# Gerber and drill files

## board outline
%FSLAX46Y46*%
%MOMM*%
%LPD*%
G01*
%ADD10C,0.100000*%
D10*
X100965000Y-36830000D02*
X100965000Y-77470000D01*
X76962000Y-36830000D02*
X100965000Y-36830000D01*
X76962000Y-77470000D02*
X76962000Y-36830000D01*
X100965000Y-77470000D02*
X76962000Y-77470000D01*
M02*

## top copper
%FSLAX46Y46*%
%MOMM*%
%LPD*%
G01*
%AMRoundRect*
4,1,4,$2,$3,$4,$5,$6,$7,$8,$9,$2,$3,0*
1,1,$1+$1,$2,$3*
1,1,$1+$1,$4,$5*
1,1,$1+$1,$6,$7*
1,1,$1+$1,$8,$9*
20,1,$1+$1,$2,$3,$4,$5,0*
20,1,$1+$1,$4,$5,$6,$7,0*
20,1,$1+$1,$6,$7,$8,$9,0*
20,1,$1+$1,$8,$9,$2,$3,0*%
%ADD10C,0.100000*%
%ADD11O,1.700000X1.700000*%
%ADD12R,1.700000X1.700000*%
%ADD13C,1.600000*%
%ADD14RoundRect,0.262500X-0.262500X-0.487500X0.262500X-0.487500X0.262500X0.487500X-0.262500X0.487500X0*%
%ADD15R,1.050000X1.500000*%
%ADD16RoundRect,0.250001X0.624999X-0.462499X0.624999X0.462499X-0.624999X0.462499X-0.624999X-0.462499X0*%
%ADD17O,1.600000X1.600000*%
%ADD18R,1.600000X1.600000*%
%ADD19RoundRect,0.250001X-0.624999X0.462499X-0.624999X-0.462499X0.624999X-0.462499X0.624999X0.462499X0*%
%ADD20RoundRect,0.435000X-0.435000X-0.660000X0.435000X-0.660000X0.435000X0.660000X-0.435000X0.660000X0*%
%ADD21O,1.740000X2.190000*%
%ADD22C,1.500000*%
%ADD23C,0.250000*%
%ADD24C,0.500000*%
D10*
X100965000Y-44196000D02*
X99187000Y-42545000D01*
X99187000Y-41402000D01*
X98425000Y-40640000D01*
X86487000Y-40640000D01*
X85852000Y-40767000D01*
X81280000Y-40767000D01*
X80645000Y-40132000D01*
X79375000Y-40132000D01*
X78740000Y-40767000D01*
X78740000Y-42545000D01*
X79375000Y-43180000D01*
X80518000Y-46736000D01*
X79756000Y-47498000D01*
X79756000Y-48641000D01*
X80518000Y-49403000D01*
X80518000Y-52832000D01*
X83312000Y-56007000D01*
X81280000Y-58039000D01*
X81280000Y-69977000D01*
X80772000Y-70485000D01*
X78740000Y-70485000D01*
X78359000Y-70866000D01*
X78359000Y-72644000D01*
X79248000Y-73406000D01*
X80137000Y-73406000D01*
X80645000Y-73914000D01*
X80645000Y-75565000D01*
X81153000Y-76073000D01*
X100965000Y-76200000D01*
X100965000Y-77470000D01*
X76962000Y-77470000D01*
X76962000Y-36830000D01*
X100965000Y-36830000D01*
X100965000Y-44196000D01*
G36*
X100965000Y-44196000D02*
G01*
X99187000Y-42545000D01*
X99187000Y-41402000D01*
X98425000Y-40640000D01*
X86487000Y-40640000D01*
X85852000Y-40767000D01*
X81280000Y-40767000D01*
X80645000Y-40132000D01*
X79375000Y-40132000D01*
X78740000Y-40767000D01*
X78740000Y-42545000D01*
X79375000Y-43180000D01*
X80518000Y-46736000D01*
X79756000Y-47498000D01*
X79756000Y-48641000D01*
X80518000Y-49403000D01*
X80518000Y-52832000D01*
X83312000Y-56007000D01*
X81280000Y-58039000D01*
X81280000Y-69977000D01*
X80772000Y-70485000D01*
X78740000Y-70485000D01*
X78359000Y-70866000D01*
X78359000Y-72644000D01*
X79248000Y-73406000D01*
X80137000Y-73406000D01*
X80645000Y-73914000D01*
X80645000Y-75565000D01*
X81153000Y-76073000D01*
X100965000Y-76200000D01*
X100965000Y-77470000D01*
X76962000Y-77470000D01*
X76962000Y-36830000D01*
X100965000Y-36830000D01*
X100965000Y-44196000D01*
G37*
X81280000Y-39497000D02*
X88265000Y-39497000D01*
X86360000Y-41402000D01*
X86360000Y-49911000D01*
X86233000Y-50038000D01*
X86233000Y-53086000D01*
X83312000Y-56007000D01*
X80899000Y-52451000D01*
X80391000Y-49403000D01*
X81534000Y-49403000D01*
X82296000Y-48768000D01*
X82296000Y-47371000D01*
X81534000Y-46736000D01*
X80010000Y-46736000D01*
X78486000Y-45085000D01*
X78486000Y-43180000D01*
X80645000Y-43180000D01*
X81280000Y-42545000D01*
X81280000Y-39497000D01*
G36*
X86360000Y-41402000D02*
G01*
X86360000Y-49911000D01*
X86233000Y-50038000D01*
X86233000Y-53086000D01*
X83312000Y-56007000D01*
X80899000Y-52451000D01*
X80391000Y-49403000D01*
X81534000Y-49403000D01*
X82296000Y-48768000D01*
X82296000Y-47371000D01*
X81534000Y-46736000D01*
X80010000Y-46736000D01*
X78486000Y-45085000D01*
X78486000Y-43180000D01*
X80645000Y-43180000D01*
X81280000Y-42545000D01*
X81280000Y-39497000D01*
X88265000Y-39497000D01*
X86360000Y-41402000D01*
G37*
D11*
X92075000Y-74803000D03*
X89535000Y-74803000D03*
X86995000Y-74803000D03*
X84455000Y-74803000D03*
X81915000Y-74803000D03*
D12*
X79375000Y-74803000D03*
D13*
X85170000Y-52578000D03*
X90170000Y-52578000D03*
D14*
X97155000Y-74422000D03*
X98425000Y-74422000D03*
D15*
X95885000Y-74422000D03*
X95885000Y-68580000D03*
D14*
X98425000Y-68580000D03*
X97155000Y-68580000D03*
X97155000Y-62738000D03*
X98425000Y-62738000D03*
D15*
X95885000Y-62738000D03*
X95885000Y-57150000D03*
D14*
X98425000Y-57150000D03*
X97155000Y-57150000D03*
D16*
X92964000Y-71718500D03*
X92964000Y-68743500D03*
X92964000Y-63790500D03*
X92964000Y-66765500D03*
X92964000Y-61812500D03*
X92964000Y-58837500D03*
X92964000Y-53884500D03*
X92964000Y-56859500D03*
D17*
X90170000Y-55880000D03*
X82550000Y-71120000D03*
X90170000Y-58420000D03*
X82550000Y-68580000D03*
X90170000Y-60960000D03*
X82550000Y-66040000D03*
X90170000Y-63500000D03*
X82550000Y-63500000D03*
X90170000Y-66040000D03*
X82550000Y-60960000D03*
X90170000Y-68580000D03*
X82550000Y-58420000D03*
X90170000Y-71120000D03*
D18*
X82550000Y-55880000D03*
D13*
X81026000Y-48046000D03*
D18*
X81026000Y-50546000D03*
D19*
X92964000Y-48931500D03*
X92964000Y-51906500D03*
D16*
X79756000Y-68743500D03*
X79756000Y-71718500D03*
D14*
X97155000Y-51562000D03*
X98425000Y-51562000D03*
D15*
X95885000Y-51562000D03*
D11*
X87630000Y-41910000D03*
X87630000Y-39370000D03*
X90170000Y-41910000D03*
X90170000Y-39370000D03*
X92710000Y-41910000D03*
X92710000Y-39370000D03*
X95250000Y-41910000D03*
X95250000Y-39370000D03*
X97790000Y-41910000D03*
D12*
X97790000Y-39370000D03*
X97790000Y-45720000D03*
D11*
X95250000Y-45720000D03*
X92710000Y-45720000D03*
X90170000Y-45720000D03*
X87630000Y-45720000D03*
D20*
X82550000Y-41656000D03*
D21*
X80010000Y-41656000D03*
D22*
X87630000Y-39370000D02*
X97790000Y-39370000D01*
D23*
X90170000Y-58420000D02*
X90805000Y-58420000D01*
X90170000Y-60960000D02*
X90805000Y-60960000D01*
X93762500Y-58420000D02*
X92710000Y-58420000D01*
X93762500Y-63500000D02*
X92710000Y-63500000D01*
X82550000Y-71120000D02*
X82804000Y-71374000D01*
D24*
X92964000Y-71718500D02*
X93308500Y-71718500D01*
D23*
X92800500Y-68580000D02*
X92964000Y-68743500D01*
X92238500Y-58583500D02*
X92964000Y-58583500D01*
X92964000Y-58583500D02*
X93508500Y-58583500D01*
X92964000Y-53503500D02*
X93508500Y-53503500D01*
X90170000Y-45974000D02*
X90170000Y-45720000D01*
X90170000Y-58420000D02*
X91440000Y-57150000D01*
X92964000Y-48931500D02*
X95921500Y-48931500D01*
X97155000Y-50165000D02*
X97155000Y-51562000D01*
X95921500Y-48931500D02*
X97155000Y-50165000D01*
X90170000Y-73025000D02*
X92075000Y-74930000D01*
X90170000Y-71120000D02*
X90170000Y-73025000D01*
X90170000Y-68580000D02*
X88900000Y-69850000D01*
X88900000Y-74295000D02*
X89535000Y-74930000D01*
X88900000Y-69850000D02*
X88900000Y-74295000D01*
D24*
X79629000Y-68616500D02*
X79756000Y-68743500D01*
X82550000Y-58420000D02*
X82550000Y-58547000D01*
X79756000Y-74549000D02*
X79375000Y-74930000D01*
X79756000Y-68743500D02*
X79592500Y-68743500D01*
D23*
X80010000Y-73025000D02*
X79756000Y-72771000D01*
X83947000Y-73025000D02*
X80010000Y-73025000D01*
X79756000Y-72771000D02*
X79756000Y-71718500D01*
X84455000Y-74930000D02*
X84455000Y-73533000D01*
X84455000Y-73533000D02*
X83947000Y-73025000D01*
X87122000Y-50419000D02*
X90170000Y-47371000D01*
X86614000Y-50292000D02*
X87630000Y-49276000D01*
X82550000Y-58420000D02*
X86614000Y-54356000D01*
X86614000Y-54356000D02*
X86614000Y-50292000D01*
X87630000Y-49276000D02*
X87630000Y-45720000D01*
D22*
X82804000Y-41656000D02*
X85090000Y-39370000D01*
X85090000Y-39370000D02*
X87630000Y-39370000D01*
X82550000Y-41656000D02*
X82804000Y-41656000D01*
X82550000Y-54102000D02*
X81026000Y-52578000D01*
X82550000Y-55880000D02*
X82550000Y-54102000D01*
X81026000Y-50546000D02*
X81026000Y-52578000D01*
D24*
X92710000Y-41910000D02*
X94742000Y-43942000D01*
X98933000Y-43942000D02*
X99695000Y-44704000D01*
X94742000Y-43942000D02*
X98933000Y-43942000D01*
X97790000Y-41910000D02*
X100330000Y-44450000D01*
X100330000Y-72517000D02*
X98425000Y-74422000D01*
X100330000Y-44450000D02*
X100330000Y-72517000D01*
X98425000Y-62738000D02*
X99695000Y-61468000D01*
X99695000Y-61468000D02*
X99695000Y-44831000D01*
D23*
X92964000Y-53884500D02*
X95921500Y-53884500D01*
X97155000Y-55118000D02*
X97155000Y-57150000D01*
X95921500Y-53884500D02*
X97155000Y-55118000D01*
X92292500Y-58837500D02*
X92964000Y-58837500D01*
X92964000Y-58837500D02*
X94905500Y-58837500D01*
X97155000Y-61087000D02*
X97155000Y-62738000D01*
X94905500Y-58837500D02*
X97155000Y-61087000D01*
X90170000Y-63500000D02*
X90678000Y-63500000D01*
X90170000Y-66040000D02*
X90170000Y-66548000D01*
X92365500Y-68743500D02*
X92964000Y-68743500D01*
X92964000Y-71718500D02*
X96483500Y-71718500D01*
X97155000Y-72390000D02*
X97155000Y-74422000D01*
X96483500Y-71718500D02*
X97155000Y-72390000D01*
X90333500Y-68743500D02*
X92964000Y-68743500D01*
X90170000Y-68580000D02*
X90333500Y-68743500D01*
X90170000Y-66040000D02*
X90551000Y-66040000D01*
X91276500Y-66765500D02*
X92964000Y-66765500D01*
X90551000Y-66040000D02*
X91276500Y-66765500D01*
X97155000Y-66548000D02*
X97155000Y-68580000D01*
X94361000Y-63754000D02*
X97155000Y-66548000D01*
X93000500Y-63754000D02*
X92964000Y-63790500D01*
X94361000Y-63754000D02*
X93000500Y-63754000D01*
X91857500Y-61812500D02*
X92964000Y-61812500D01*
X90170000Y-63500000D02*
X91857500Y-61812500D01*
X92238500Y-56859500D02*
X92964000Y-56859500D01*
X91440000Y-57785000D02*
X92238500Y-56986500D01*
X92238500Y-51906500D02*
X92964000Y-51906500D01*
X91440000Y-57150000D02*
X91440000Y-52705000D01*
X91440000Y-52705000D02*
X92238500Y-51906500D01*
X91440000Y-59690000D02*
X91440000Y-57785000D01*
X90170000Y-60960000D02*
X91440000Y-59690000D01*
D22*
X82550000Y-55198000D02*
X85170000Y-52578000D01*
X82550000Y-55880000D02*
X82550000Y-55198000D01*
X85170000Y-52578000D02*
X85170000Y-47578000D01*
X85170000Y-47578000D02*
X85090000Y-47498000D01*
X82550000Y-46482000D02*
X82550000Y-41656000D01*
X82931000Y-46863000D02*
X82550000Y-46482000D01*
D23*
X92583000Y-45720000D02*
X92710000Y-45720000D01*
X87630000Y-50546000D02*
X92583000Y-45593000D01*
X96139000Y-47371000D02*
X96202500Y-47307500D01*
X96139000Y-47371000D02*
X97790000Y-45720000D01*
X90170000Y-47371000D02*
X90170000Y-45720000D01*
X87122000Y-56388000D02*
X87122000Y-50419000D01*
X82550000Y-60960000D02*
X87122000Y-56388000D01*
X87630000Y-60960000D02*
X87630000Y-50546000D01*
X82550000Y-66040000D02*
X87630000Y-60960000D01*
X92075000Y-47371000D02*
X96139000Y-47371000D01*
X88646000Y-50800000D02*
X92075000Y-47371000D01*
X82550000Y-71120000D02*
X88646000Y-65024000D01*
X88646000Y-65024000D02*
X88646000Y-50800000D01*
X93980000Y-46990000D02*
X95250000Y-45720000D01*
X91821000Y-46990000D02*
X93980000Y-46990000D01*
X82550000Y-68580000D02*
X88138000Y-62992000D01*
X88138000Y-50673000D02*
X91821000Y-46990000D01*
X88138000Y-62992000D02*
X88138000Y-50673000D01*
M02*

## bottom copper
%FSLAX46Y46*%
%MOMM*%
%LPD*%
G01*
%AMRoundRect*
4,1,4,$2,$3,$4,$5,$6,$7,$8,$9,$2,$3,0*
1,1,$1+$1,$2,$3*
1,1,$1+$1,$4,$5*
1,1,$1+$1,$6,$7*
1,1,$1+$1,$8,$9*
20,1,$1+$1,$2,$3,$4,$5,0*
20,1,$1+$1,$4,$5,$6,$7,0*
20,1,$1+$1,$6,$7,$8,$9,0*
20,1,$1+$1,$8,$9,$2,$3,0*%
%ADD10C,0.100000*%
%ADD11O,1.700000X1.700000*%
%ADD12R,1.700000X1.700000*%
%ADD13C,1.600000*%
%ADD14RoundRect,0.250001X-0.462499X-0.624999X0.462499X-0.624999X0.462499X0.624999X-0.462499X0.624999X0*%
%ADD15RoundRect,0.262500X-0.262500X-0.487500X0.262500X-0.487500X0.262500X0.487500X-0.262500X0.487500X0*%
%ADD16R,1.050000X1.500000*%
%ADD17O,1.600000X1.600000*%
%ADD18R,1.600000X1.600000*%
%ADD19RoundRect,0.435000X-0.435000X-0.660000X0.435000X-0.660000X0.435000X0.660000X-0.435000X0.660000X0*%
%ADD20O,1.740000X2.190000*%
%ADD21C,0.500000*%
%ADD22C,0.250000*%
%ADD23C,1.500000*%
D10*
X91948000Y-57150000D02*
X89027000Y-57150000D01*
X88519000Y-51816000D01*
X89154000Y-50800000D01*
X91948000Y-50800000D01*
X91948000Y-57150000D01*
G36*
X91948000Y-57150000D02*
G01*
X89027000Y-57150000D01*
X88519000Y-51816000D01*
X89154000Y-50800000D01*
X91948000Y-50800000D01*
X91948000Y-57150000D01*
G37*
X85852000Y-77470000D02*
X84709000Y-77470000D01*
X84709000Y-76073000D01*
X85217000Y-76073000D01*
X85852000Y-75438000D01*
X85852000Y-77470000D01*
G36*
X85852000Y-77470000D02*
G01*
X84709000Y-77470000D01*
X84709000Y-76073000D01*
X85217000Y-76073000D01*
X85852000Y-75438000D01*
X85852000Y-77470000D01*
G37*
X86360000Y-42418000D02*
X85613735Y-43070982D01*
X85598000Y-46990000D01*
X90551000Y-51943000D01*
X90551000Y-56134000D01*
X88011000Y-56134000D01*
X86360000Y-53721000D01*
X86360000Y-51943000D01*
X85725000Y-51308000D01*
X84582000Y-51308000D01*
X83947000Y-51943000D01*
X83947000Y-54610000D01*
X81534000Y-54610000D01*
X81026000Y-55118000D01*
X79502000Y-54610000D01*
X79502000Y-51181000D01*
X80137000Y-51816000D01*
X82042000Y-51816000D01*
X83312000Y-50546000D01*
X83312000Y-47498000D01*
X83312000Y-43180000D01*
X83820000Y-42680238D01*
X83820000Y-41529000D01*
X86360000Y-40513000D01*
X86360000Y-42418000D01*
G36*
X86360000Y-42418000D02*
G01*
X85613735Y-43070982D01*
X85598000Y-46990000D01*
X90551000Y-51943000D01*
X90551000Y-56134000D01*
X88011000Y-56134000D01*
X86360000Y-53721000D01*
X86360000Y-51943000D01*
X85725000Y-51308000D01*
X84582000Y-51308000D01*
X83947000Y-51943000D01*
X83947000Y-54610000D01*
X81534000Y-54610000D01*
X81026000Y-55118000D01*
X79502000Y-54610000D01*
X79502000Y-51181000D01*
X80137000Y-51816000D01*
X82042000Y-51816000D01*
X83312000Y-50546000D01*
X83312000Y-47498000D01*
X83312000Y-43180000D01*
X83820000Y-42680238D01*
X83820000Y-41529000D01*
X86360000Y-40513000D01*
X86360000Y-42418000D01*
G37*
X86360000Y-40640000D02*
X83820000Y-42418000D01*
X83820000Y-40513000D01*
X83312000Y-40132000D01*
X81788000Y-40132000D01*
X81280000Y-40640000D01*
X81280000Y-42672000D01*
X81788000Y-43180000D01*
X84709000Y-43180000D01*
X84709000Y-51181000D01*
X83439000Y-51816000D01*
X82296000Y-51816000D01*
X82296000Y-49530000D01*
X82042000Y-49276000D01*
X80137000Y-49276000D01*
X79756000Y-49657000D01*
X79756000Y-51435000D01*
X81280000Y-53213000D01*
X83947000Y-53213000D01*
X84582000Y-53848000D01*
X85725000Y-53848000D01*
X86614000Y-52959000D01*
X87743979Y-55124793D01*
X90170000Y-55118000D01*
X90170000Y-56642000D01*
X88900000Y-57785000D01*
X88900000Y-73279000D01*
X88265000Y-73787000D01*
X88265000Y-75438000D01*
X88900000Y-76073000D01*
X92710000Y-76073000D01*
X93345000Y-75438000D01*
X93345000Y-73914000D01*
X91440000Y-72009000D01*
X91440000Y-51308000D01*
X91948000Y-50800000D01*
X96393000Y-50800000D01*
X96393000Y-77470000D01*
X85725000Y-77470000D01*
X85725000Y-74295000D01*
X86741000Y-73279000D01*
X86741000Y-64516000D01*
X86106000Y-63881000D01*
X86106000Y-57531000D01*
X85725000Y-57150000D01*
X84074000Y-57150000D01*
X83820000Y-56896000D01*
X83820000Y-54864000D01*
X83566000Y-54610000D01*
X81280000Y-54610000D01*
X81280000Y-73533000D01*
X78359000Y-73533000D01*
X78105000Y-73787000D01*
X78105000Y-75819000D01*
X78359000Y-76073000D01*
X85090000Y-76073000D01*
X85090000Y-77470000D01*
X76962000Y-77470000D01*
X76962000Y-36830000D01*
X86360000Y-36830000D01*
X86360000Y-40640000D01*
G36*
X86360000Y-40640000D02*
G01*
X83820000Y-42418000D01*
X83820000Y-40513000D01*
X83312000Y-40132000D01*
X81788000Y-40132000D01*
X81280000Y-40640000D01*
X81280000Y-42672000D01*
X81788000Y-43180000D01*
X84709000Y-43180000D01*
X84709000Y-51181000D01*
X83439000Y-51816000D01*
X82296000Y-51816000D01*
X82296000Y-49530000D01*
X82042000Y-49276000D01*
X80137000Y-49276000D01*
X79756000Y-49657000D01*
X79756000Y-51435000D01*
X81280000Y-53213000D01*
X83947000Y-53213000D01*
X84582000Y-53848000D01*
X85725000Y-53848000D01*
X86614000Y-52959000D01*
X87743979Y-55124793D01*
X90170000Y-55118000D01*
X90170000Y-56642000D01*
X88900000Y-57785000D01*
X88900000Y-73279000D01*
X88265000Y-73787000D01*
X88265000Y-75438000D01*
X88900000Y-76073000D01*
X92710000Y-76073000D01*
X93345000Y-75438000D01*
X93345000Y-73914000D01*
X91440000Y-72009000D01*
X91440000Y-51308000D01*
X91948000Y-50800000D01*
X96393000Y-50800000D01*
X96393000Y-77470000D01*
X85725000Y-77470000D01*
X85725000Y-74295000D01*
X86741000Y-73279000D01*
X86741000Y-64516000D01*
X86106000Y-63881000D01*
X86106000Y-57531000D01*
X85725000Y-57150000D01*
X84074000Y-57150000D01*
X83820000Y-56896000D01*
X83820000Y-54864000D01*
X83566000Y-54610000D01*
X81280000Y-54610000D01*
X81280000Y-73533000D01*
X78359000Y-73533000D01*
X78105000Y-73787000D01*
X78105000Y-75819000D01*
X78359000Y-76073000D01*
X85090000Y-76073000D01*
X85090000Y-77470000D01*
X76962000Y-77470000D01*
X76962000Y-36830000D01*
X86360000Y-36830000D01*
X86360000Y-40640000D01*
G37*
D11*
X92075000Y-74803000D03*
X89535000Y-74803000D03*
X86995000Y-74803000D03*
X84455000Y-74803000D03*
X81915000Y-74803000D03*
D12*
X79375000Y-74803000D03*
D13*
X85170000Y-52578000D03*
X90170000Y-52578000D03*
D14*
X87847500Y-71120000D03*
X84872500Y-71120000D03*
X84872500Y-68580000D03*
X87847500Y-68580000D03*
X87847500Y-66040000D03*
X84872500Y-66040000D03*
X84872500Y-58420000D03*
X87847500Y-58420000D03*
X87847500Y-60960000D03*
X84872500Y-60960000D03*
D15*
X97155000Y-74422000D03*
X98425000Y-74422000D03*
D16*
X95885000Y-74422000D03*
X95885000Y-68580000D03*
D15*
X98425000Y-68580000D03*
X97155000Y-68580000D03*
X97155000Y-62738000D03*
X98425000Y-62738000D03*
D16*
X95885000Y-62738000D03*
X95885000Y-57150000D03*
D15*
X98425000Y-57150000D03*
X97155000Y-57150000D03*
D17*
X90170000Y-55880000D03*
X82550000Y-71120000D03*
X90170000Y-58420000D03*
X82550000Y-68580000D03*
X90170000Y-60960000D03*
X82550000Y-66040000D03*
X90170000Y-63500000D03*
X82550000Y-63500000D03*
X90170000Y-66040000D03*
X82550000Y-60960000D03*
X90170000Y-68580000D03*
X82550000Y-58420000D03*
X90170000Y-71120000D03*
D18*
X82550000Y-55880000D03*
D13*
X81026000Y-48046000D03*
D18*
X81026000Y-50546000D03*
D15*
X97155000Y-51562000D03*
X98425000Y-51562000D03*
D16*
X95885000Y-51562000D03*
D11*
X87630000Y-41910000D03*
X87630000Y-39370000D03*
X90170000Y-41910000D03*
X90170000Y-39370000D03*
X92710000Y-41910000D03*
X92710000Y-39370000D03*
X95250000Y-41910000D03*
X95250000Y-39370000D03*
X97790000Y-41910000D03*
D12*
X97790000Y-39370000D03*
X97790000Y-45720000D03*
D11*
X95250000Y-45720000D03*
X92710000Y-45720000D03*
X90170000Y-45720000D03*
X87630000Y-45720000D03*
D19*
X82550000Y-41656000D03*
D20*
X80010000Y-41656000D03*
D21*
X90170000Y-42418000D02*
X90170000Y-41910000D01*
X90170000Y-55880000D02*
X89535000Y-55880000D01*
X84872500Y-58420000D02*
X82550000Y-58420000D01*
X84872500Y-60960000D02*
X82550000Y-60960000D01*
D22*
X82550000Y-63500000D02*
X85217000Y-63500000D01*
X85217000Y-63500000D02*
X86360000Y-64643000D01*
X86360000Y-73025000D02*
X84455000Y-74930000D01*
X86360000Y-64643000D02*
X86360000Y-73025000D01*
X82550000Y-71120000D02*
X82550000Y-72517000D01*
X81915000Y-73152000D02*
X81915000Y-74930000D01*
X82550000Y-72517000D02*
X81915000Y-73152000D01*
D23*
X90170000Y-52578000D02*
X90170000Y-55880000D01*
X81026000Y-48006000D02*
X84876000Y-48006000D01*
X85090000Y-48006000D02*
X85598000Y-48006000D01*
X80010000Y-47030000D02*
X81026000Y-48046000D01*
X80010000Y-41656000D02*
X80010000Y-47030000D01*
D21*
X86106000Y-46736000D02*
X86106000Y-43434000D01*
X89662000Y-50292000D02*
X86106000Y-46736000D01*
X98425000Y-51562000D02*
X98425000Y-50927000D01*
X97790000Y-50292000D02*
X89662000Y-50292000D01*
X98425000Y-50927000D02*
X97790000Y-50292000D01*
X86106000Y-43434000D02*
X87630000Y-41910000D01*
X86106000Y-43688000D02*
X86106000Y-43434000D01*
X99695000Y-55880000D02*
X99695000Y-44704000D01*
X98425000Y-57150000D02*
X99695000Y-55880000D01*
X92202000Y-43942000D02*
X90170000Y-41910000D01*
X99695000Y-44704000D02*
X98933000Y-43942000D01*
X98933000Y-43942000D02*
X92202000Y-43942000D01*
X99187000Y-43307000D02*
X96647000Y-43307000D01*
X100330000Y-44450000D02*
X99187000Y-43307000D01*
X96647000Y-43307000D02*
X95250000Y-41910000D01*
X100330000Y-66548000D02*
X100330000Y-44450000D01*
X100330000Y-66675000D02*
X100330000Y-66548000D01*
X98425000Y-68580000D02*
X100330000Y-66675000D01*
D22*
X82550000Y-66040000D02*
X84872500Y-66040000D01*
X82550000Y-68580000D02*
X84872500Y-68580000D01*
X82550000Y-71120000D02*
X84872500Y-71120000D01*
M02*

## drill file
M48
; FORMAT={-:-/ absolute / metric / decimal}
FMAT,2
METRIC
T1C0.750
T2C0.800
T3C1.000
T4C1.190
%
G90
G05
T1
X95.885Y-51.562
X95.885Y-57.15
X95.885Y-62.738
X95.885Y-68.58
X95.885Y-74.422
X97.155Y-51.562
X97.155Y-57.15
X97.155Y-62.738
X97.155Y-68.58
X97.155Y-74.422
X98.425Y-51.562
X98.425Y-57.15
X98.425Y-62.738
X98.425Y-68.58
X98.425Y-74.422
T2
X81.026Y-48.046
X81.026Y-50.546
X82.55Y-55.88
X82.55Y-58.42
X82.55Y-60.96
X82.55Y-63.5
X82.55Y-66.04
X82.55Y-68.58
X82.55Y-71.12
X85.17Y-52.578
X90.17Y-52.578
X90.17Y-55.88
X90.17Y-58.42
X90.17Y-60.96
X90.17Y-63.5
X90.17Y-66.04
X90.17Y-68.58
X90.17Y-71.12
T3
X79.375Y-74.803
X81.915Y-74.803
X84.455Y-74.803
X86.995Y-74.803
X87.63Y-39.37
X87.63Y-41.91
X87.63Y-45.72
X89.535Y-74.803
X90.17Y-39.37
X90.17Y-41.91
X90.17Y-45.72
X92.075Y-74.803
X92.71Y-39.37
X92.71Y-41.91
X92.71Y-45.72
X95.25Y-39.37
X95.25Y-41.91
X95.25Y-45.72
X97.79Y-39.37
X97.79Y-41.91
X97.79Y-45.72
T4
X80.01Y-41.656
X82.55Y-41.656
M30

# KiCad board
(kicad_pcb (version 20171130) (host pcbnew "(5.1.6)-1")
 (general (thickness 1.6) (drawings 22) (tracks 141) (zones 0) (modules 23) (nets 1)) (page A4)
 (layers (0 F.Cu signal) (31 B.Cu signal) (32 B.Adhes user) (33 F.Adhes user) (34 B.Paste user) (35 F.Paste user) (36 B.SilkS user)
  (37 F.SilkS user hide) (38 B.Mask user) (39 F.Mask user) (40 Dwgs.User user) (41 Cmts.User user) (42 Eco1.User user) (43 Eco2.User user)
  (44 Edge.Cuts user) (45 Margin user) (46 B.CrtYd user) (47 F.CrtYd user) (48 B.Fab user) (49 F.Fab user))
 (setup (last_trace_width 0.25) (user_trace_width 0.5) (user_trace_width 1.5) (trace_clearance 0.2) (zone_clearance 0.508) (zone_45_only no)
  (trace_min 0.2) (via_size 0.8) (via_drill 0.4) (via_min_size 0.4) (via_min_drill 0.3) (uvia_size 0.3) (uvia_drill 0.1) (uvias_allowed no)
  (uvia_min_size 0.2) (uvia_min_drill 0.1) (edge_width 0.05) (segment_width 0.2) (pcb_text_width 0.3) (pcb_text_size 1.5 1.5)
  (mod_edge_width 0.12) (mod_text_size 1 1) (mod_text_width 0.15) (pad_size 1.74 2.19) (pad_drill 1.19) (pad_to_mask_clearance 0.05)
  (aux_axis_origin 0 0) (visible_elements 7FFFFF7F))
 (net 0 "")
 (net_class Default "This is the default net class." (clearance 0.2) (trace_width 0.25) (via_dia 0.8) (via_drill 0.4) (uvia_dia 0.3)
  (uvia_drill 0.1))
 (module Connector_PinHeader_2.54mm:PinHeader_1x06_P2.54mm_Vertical (layer F.Cu) (at 79.375 74.803 90)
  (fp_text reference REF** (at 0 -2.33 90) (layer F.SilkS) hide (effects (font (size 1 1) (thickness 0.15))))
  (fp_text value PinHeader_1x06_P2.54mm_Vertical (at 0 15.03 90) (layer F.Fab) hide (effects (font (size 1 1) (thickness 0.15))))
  (pad 6 thru_hole oval (at 0 12.7 90) (size 1.7 1.7) (drill 1) (layers *.Cu *.Mask))
  (pad 5 thru_hole oval (at 0 10.16 90) (size 1.7 1.7) (drill 1) (layers *.Cu *.Mask))
  (pad 4 thru_hole oval (at 0 7.62 90) (size 1.7 1.7) (drill 1) (layers *.Cu *.Mask))
  (pad 3 thru_hole oval (at 0 5.08 90) (size 1.7 1.7) (drill 1) (layers *.Cu *.Mask))
  (pad 2 thru_hole oval (at 0 2.54 90) (size 1.7 1.7) (drill 1) (layers *.Cu *.Mask))
  (pad 1 thru_hole rect (at 0 0 90) (size 1.7 1.7) (drill 1) (layers *.Cu *.Mask)))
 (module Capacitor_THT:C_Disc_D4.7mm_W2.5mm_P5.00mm (layer F.Cu) (at 90.17 52.578 180)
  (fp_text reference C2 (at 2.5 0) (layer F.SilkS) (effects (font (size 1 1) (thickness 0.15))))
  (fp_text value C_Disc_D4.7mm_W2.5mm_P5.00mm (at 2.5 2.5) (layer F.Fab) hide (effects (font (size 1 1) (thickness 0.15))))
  (pad 2 thru_hole circle (at 5 0 180) (size 1.6 1.6) (drill 0.8) (layers *.Cu *.Mask))
  (pad 1 thru_hole circle (at 0 0 180) (size 1.6 1.6) (drill 0.8) (layers *.Cu *.Mask)))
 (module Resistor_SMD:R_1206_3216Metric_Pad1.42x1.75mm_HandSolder (layer B.Cu) (at 86.36 71.12)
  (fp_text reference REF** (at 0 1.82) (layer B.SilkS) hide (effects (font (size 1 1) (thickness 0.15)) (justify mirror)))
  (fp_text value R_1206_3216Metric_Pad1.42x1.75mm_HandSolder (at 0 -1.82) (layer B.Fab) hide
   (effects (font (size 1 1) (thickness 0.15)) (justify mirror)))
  (pad 2 smd roundrect (at 1.4875 0) (size 1.425 1.75) (layers B.Cu B.Paste B.Mask) (roundrect_rratio 0.175439))
  (pad 1 smd roundrect (at -1.4875 0) (size 1.425 1.75) (layers B.Cu B.Paste B.Mask) (roundrect_rratio 0.175439)))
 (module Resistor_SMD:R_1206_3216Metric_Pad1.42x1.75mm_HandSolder (layer B.Cu) (at 86.36 68.58)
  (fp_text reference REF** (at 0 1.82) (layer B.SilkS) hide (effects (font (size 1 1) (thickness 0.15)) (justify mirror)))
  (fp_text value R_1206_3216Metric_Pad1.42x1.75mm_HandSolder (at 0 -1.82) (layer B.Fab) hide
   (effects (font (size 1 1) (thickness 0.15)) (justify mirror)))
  (pad 1 smd roundrect (at -1.4875 0) (size 1.425 1.75) (layers B.Cu B.Paste B.Mask) (roundrect_rratio 0.175439))
  (pad 2 smd roundrect (at 1.4875 0) (size 1.425 1.75) (layers B.Cu B.Paste B.Mask) (roundrect_rratio 0.175439)))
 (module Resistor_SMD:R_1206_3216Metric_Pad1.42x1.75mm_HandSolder (layer B.Cu) (at 86.36 66.04)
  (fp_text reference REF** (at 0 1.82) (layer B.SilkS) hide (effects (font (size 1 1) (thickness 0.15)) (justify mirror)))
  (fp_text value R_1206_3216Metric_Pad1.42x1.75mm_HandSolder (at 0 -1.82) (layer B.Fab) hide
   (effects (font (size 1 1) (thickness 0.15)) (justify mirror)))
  (pad 2 smd roundrect (at 1.4875 0) (size 1.425 1.75) (layers B.Cu B.Paste B.Mask) (roundrect_rratio 0.175439))
  (pad 1 smd roundrect (at -1.4875 0) (size 1.425 1.75) (layers B.Cu B.Paste B.Mask) (roundrect_rratio 0.175439)))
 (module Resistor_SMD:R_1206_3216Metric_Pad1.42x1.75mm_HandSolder (layer B.Cu) (at 86.36 58.42)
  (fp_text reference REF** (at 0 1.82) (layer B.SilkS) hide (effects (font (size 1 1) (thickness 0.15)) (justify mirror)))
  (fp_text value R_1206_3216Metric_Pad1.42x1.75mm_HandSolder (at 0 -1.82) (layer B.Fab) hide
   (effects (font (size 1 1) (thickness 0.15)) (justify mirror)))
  (pad 1 smd roundrect (at -1.4875 0) (size 1.425 1.75) (layers B.Cu B.Paste B.Mask) (roundrect_rratio 0.175439))
  (pad 2 smd roundrect (at 1.4875 0) (size 1.425 1.75) (layers B.Cu B.Paste B.Mask) (roundrect_rratio 0.175439)))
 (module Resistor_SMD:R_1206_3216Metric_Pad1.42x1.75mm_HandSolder (layer B.Cu) (at 86.36 60.96)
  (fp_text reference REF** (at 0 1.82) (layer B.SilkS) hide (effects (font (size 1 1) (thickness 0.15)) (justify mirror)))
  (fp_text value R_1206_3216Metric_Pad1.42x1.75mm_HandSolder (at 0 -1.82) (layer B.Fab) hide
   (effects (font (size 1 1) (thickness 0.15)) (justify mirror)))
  (pad 2 smd roundrect (at 1.4875 0) (size 1.425 1.75) (layers B.Cu B.Paste B.Mask) (roundrect_rratio 0.175439))
  (pad 1 smd roundrect (at -1.4875 0) (size 1.425 1.75) (layers B.Cu B.Paste B.Mask) (roundrect_rratio 0.175439)))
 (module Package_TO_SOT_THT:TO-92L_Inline (layer F.Cu) (at 95.885 74.422)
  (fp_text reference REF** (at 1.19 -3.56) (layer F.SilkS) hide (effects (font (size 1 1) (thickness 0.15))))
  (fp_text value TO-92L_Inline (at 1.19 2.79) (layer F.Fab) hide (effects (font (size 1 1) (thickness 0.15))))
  (pad 2 thru_hole roundrect (at 1.27 0) (size 1.05 1.5) (drill 0.75) (layers *.Cu *.Mask) (roundrect_rratio 0.25))
  (pad 3 thru_hole roundrect (at 2.54 0) (size 1.05 1.5) (drill 0.75) (layers *.Cu *.Mask) (roundrect_rratio 0.25))
  (pad 1 thru_hole rect (at 0 0) (size 1.05 1.5) (drill 0.75) (layers *.Cu *.Mask)))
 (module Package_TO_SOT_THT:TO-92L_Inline (layer F.Cu) (at 95.885 68.58)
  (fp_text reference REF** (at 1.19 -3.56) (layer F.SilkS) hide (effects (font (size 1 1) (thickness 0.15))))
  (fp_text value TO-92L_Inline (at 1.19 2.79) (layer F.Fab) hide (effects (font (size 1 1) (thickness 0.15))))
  (pad 1 thru_hole rect (at 0 0) (size 1.05 1.5) (drill 0.75) (layers *.Cu *.Mask))
  (pad 3 thru_hole roundrect (at 2.54 0) (size 1.05 1.5) (drill 0.75) (layers *.Cu *.Mask) (roundrect_rratio 0.25))
  (pad 2 thru_hole roundrect (at 1.27 0) (size 1.05 1.5) (drill 0.75) (layers *.Cu *.Mask) (roundrect_rratio 0.25)))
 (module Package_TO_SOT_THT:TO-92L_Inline (layer F.Cu) (at 95.885 62.738)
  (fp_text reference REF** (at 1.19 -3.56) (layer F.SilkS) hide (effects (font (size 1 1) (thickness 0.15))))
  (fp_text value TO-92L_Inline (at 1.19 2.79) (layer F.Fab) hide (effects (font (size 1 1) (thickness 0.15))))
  (pad 2 thru_hole roundrect (at 1.27 0) (size 1.05 1.5) (drill 0.75) (layers *.Cu *.Mask) (roundrect_rratio 0.25))
  (pad 3 thru_hole roundrect (at 2.54 0) (size 1.05 1.5) (drill 0.75) (layers *.Cu *.Mask) (roundrect_rratio 0.25))
  (pad 1 thru_hole rect (at 0 0) (size 1.05 1.5) (drill 0.75) (layers *.Cu *.Mask)))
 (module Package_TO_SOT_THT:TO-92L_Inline (layer F.Cu) (at 95.885 57.15)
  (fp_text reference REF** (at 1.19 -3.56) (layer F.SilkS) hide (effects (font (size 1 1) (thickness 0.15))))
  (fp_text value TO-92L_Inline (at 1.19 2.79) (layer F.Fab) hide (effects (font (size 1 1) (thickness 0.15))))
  (pad 1 thru_hole rect (at 0 0) (size 1.05 1.5) (drill 0.75) (layers *.Cu *.Mask))
  (pad 3 thru_hole roundrect (at 2.54 0) (size 1.05 1.5) (drill 0.75) (layers *.Cu *.Mask) (roundrect_rratio 0.25))
  (pad 2 thru_hole roundrect (at 1.27 0) (size 1.05 1.5) (drill 0.75) (layers *.Cu *.Mask) (roundrect_rratio 0.25)))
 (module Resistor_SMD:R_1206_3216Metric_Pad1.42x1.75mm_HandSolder (layer F.Cu) (at 92.964 70.231 90)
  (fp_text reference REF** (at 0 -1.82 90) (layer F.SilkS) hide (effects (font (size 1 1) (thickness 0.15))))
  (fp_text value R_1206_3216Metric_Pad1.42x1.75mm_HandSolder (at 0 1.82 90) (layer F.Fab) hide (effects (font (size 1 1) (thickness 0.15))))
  (pad 1 smd roundrect (at -1.4875 0 90) (size 1.425 1.75) (layers F.Cu F.Paste F.Mask) (roundrect_rratio 0.175439))
  (pad 2 smd roundrect (at 1.4875 0 90) (size 1.425 1.75) (layers F.Cu F.Paste F.Mask) (roundrect_rratio 0.175439)))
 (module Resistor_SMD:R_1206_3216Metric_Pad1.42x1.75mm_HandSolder (layer F.Cu) (at 92.964 65.278 90)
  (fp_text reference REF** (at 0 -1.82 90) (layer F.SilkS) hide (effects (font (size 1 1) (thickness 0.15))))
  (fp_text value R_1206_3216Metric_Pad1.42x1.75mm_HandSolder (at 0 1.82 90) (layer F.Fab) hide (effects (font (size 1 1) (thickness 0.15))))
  (pad 2 smd roundrect (at 1.4875 0 90) (size 1.425 1.75) (layers F.Cu F.Paste F.Mask) (roundrect_rratio 0.175439))
  (pad 1 smd roundrect (at -1.4875 0 90) (size 1.425 1.75) (layers F.Cu F.Paste F.Mask) (roundrect_rratio 0.175439)))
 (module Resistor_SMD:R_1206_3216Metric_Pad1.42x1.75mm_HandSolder (layer F.Cu) (at 92.964 60.325 90)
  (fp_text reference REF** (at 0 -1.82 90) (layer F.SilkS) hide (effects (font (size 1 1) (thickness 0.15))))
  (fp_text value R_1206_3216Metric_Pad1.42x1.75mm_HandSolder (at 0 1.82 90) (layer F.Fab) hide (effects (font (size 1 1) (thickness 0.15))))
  (pad 1 smd roundrect (at -1.4875 0 90) (size 1.425 1.75) (layers F.Cu F.Paste F.Mask) (roundrect_rratio 0.175439))
  (pad 2 smd roundrect (at 1.4875 0 90) (size 1.425 1.75) (layers F.Cu F.Paste F.Mask) (roundrect_rratio 0.175439)))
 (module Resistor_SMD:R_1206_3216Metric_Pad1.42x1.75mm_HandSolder (layer F.Cu) (at 92.964 55.372 90)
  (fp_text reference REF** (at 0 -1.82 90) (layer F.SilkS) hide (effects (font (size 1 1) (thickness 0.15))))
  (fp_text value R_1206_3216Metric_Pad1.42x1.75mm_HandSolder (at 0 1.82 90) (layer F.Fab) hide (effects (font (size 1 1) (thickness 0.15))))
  (pad 2 smd roundrect (at 1.4875 0 90) (size 1.425 1.75) (layers F.Cu F.Paste F.Mask) (roundrect_rratio 0.175439))
  (pad 1 smd roundrect (at -1.4875 0 90) (size 1.425 1.75) (layers F.Cu F.Paste F.Mask) (roundrect_rratio 0.175439)))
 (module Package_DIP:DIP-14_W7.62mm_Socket (layer F.Cu) (at 82.55 55.88)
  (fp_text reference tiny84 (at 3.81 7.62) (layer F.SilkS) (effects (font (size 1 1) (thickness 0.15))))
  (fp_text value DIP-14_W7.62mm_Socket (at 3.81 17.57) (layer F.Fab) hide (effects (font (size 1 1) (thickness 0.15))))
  (pad 14 thru_hole oval (at 7.62 0) (size 1.6 1.6) (drill 0.8) (layers *.Cu *.Mask))
  (pad 7 thru_hole oval (at 0 15.24) (size 1.6 1.6) (drill 0.8) (layers *.Cu *.Mask))
  (pad 13 thru_hole oval (at 7.62 2.54) (size 1.6 1.6) (drill 0.8) (layers *.Cu *.Mask))
  (pad 6 thru_hole oval (at 0 12.7) (size 1.6 1.6) (drill 0.8) (layers *.Cu *.Mask))
  (pad 12 thru_hole oval (at 7.62 5.08) (size 1.6 1.6) (drill 0.8) (layers *.Cu *.Mask))
  (pad 5 thru_hole oval (at 0 10.16) (size 1.6 1.6) (drill 0.8) (layers *.Cu *.Mask))
  (pad 11 thru_hole oval (at 7.62 7.62) (size 1.6 1.6) (drill 0.8) (layers *.Cu *.Mask))
  (pad 4 thru_hole oval (at 0 7.62) (size 1.6 1.6) (drill 0.8) (layers *.Cu *.Mask))
  (pad 10 thru_hole oval (at 7.62 10.16) (size 1.6 1.6) (drill 0.8) (layers *.Cu *.Mask))
  (pad 3 thru_hole oval (at 0 5.08) (size 1.6 1.6) (drill 0.8) (layers *.Cu *.Mask))
  (pad 9 thru_hole oval (at 7.62 12.7) (size 1.6 1.6) (drill 0.8) (layers *.Cu *.Mask))
  (pad 2 thru_hole oval (at 0 2.54) (size 1.6 1.6) (drill 0.8) (layers *.Cu *.Mask))
  (pad 8 thru_hole oval (at 7.62 15.24) (size 1.6 1.6) (drill 0.8) (layers *.Cu *.Mask))
  (pad 1 thru_hole rect (at 0 0) (size 1.6 1.6) (drill 0.8) (layers *.Cu *.Mask)))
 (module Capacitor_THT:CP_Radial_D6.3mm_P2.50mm (layer F.Cu) (at 81.026 50.546 90)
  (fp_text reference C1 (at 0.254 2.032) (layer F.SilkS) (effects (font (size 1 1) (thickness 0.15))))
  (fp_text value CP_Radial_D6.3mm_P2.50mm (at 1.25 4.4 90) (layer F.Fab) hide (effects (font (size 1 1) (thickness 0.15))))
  (pad 2 thru_hole circle (at 2.5 0 90) (size 1.6 1.6) (drill 0.8) (layers *.Cu *.Mask))
  (pad 1 thru_hole rect (at 0 0 90) (size 1.6 1.6) (drill 0.8) (layers *.Cu *.Mask)))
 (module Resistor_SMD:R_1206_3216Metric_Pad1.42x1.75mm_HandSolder (layer F.Cu) (at 92.964 50.419 270)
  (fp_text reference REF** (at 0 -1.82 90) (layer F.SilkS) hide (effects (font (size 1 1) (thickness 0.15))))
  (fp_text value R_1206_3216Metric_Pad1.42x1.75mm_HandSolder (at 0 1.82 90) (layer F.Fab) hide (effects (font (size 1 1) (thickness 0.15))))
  (pad 1 smd roundrect (at -1.4875 0 270) (size 1.425 1.75) (layers F.Cu F.Paste F.Mask) (roundrect_rratio 0.175439))
  (pad 2 smd roundrect (at 1.4875 0 270) (size 1.425 1.75) (layers F.Cu F.Paste F.Mask) (roundrect_rratio 0.175439)))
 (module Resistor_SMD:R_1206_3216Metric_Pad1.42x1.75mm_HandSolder (layer F.Cu) (at 79.756 70.231 90)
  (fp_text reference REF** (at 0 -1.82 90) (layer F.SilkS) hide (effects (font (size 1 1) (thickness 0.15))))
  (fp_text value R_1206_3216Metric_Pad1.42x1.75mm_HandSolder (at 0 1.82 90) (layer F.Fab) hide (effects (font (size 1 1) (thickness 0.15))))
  (pad 2 smd roundrect (at 1.4875 0 90) (size 1.425 1.75) (layers F.Cu F.Paste F.Mask) (roundrect_rratio 0.175439))
  (pad 1 smd roundrect (at -1.4875 0 90) (size 1.425 1.75) (layers F.Cu F.Paste F.Mask) (roundrect_rratio 0.175439)))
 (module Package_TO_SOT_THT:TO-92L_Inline (layer F.Cu) (at 95.885 51.562)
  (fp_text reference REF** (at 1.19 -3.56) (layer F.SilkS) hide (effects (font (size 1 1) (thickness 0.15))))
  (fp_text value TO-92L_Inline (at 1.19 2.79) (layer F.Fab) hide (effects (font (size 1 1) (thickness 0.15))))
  (pad 2 thru_hole roundrect (at 1.27 0) (size 1.05 1.5) (drill 0.75) (layers *.Cu *.Mask) (roundrect_rratio 0.25))
  (pad 3 thru_hole roundrect (at 2.54 0) (size 1.05 1.5) (drill 0.75) (layers *.Cu *.Mask) (roundrect_rratio 0.25))
  (pad 1 thru_hole rect (at 0 0) (size 1.05 1.5) (drill 0.75) (layers *.Cu *.Mask)))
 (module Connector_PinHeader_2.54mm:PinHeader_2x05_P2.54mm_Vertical (layer F.Cu) (at 97.79 39.37 270)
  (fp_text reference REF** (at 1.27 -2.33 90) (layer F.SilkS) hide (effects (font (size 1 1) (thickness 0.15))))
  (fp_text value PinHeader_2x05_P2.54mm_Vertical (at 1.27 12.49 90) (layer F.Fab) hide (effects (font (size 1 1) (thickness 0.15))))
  (pad 10 thru_hole oval (at 2.54 10.16 270) (size 1.7 1.7) (drill 1) (layers *.Cu *.Mask))
  (pad 9 thru_hole oval (at 0 10.16 270) (size 1.7 1.7) (drill 1) (layers *.Cu *.Mask))
  (pad 8 thru_hole oval (at 2.54 7.62 270) (size 1.7 1.7) (drill 1) (layers *.Cu *.Mask))
  (pad 7 thru_hole oval (at 0 7.62 270) (size 1.7 1.7) (drill 1) (layers *.Cu *.Mask))
  (pad 6 thru_hole oval (at 2.54 5.08 270) (size 1.7 1.7) (drill 1) (layers *.Cu *.Mask))
  (pad 5 thru_hole oval (at 0 5.08 270) (size 1.7 1.7) (drill 1) (layers *.Cu *.Mask))
  (pad 4 thru_hole oval (at 2.54 2.54 270) (size 1.7 1.7) (drill 1) (layers *.Cu *.Mask))
  (pad 3 thru_hole oval (at 0 2.54 270) (size 1.7 1.7) (drill 1) (layers *.Cu *.Mask))
  (pad 2 thru_hole oval (at 2.54 0 270) (size 1.7 1.7) (drill 1) (layers *.Cu *.Mask))
  (pad 1 thru_hole rect (at 0 0 270) (size 1.7 1.7) (drill 1) (layers *.Cu *.Mask)))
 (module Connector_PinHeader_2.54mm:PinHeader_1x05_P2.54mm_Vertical (layer F.Cu) (at 97.79 45.72 270)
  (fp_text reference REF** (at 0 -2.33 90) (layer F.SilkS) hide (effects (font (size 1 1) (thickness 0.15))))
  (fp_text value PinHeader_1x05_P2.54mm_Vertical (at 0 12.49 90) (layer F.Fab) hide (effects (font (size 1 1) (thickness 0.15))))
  (pad 1 thru_hole rect (at 0 0 270) (size 1.7 1.7) (drill 1) (layers *.Cu *.Mask))
  (pad 2 thru_hole oval (at 0 2.54 270) (size 1.7 1.7) (drill 1) (layers *.Cu *.Mask))
  (pad 3 thru_hole oval (at 0 5.08 270) (size 1.7 1.7) (drill 1) (layers *.Cu *.Mask))
  (pad 4 thru_hole oval (at 0 7.62 270) (size 1.7 1.7) (drill 1) (layers *.Cu *.Mask))
  (pad 5 thru_hole oval (at 0 10.16 270) (size 1.7 1.7) (drill 1) (layers *.Cu *.Mask)))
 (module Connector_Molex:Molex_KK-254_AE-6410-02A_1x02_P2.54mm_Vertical (layer F.Cu) (at 80.01 41.656)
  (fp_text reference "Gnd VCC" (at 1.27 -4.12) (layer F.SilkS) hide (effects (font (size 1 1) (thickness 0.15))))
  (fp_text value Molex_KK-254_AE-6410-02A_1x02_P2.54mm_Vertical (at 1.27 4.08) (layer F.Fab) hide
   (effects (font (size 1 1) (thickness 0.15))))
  (pad 1 thru_hole roundrect (at 2.54 0) (size 1.74 2.19) (drill 1.19) (layers *.Cu *.Mask) (roundrect_rratio 0.25))
  (pad 2 thru_hole oval (at 0 0) (size 1.74 2.19) (drill 1.19) (layers *.Cu *.Mask)))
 (gr_poly (pts (xy 91.948 57.15) (xy 89.027 57.15) (xy 88.519 51.816) (xy 89.154 50.8) (xy 91.948 50.8)) (layer B.Cu) (width 0.1))
 (gr_poly (pts (xy 85.852 77.47) (xy 84.709 77.47) (xy 84.709 76.073) (xy 85.217 76.073) (xy 85.852 75.438)) (layer B.Cu) (width 0.1))
 (gr_poly
  (pts (xy 86.36 42.418) (xy 85.613735 43.070982) (xy 85.598 46.99) (xy 90.551 51.943) (xy 90.551 56.134) (xy 88.011 56.134)
   (xy 86.36 53.721) (xy 86.36 51.943) (xy 85.725 51.308) (xy 84.582 51.308) (xy 83.947 51.943) (xy 83.947 54.61) (xy 81.534 54.61)
   (xy 81.026 55.118) (xy 79.502 54.61) (xy 79.502 51.181) (xy 80.137 51.816) (xy 82.042 51.816) (xy 83.312 50.546) (xy 83.312 47.498)
   (xy 83.312 43.18) (xy 83.82 42.680238) (xy 83.82 41.529) (xy 86.36 40.513))
  (layer B.Cu) (width 0.1))
 (gr_poly
  (pts (xy 86.36 40.64) (xy 83.82 42.418) (xy 83.82 40.513) (xy 83.312 40.132) (xy 81.788 40.132) (xy 81.28 40.64) (xy 81.28 42.672)
   (xy 81.788 43.18) (xy 84.709 43.18) (xy 84.709 51.181) (xy 83.439 51.816) (xy 82.296 51.816) (xy 82.296 49.53) (xy 82.042 49.276)
   (xy 80.137 49.276) (xy 79.756 49.657) (xy 79.756 51.435) (xy 81.28 53.213) (xy 83.947 53.213) (xy 84.582 53.848) (xy 85.725 53.848)
   (xy 86.614 52.959) (xy 87.743979 55.124793) (xy 90.17 55.118) (xy 90.17 56.642) (xy 88.9 57.785) (xy 88.9 73.279) (xy 88.265 73.787)
   (xy 88.265 75.438) (xy 88.9 76.073) (xy 92.71 76.073) (xy 93.345 75.438) (xy 93.345 73.914) (xy 91.44 72.009) (xy 91.44 51.308)
   (xy 91.948 50.8) (xy 96.393 50.8) (xy 96.393 77.47) (xy 85.725 77.47) (xy 85.725 74.295) (xy 86.741 73.279) (xy 86.741 64.516)
   (xy 86.106 63.881) (xy 86.106 57.531) (xy 85.725 57.15) (xy 84.074 57.15) (xy 83.82 56.896) (xy 83.82 54.864) (xy 83.566 54.61)
   (xy 81.28 54.61) (xy 81.28 73.533) (xy 78.359 73.533) (xy 78.105 73.787) (xy 78.105 75.819) (xy 78.359 76.073) (xy 85.09 76.073)
   (xy 85.09 77.47) (xy 76.962 77.47) (xy 76.962 36.83) (xy 86.36 36.83))
  (layer B.Cu) (width 0.1))
 (gr_poly
  (pts (xy 100.965 44.196) (xy 99.187 42.545) (xy 99.187 41.402) (xy 98.425 40.64) (xy 86.487 40.64) (xy 85.852 40.767) (xy 81.28 40.767)
   (xy 80.645 40.132) (xy 79.375 40.132) (xy 78.74 40.767) (xy 78.74 42.545) (xy 79.375 43.18) (xy 80.518 46.736) (xy 79.756 47.498)
   (xy 79.756 48.641) (xy 80.518 49.403) (xy 80.518 52.832) (xy 83.312 56.007) (xy 81.28 58.039) (xy 81.28 69.977) (xy 80.772 70.485)
   (xy 78.74 70.485) (xy 78.359 70.866) (xy 78.359 72.644) (xy 79.248 73.406) (xy 80.137 73.406) (xy 80.645 73.914) (xy 80.645 75.565)
   (xy 81.153 76.073) (xy 100.965 76.2) (xy 100.965 77.47) (xy 76.962 77.47) (xy 76.962 36.83) (xy 100.965 36.83))
  (layer F.Cu) (width 0.1))
 (gr_poly
  (pts (xy 81.28 39.497) (xy 88.265 39.497) (xy 86.36 41.402) (xy 86.36 49.911) (xy 86.233 50.038) (xy 86.233 53.086) (xy 83.312 56.007)
   (xy 80.899 52.451) (xy 80.391 49.403) (xy 81.534 49.403) (xy 82.296 48.768) (xy 82.296 47.371) (xy 81.534 46.736) (xy 80.01 46.736)
   (xy 78.486 45.085) (xy 78.486 43.18) (xy 80.645 43.18) (xy 81.28 42.545))
  (layer F.Cu) (width 0.1))
 (gr_line (start 100.965 36.83) (end 100.965 77.47) (layer Edge.Cuts) (width 0.1))
 (gr_line (start 76.962 36.83) (end 100.965 36.83) (layer Edge.Cuts) (width 0.1))
 (gr_line (start 76.962 77.47) (end 76.962 36.83) (layer Edge.Cuts) (width 0.1))
 (gr_line (start 100.965 77.47) (end 76.962 77.47) (layer Edge.Cuts) (width 0.1))
 (segment (start 87.63 39.37) (end 97.79 39.37) (width 1.5) (layer F.Cu) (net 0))
 (segment (start 90.17 58.42) (end 90.805 58.42) (width 0.25) (layer F.Cu) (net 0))
 (segment (start 90.17 60.96) (end 90.805 60.96) (width 0.25) (layer F.Cu) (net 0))
 (segment (start 93.7625 58.42) (end 92.71 58.42) (width 0.25) (layer F.Cu) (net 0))
 (segment (start 93.7625 63.5) (end 92.71 63.5) (width 0.25) (layer F.Cu) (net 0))
 (segment (start 90.17 42.418) (end 90.17 41.91) (width 0.5) (layer B.Cu) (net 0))
 (segment (start 82.55 71.12) (end 82.804 71.374) (width 0.25) (layer F.Cu) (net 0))
 (segment (start 90.17 55.88) (end 89.535 55.88) (width 0.5) (layer B.Cu) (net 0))
 (segment (start 84.8725 58.42) (end 82.55 58.42) (width 0.5) (layer B.Cu) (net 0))
 (segment (start 84.8725 60.96) (end 82.55 60.96) (width 0.5) (layer B.Cu) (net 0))
 (segment (start 92.964 71.7185) (end 93.3085 71.7185) (width 0.5) (layer F.Cu) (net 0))
 (segment (start 92.8005 68.58) (end 92.964 68.7435) (width 0.25) (layer F.Cu) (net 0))
 (segment (start 92.2385 58.5835) (end 92.964 58.5835) (width 0.25) (layer F.Cu) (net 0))
 (segment (start 92.964 58.5835) (end 93.5085 58.5835) (width 0.25) (layer F.Cu) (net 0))
 (segment (start 92.964 53.5035) (end 93.5085 53.5035) (width 0.25) (layer F.Cu) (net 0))
 (segment (start 90.17 45.974) (end 90.17 45.72) (width 0.25) (layer F.Cu) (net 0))
 (segment (start 90.17 58.42) (end 91.44 57.15) (width 0.25) (layer F.Cu) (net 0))
 (segment (start 92.964 48.9315) (end 95.9215 48.9315) (width 0.25) (layer F.Cu) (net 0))
 (segment (start 97.155 50.165) (end 97.155 51.562) (width 0.25) (layer F.Cu) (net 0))
 (segment (start 95.9215 48.9315) (end 97.155 50.165) (width 0.25) (layer F.Cu) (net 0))
 (segment (start 90.17 73.025) (end 92.075 74.93) (width 0.25) (layer F.Cu) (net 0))
 (segment (start 90.17 71.12) (end 90.17 73.025) (width 0.25) (layer F.Cu) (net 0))
 (segment (start 90.17 68.58) (end 88.9 69.85) (width 0.25) (layer F.Cu) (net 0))
 (segment (start 88.9 74.295) (end 89.535 74.93) (width 0.25) (layer F.Cu) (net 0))
 (segment (start 88.9 69.85) (end 88.9 74.295) (width 0.25) (layer F.Cu) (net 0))
 (segment (start 79.629 68.6165) (end 79.756 68.7435) (width 0.5) (layer F.Cu) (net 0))
 (segment (start 82.55 58.42) (end 82.55 58.547) (width 0.5) (layer F.Cu) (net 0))
 (segment (start 79.756 74.549) (end 79.375 74.93) (width 0.5) (layer F.Cu) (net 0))
 (segment (start 82.55 63.5) (end 85.217 63.5) (width 0.25) (layer B.Cu) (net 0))
 (segment (start 85.217 63.5) (end 86.36 64.643) (width 0.25) (layer B.Cu) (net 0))
 (segment (start 86.36 73.025) (end 84.455 74.93) (width 0.25) (layer B.Cu) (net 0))
 (segment (start 86.36 64.643) (end 86.36 73.025) (width 0.25) (layer B.Cu) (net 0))
 (segment (start 79.756 68.7435) (end 79.5925 68.7435) (width 0.5) (layer F.Cu) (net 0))
 (segment (start 82.55 71.12) (end 82.55 72.517) (width 0.25) (layer B.Cu) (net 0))
 (segment (start 81.915 73.152) (end 81.915 74.93) (width 0.25) (layer B.Cu) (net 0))
 (segment (start 82.55 72.517) (end 81.915 73.152) (width 0.25) (layer B.Cu) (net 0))
 (segment (start 80.01 73.025) (end 79.756 72.771) (width 0.25) (layer F.Cu) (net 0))
 (segment (start 83.947 73.025) (end 80.01 73.025) (width 0.25) (layer F.Cu) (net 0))
 (segment (start 79.756 72.771) (end 79.756 71.7185) (width 0.25) (layer F.Cu) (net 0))
 (segment (start 84.455 74.93) (end 84.455 73.533) (width 0.25) (layer F.Cu) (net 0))
 (segment (start 84.455 73.533) (end 83.947 73.025) (width 0.25) (layer F.Cu) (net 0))
 (segment (start 87.122 50.419) (end 90.17 47.371) (width 0.25) (layer F.Cu) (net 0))
 (segment (start 86.614 50.292) (end 87.63 49.276) (width 0.25) (layer F.Cu) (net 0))
 (segment (start 82.55 58.42) (end 86.614 54.356) (width 0.25) (layer F.Cu) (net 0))
 (segment (start 86.614 54.356) (end 86.614 50.292) (width 0.25) (layer F.Cu) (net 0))
 (segment (start 87.63 49.276) (end 87.63 45.72) (width 0.25) (layer F.Cu) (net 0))
 (segment (start 90.17 52.578) (end 90.17 55.88) (width 1.5) (layer B.Cu) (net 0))
 (segment (start 81.026 48.006) (end 84.876 48.006) (width 1.5) (layer B.Cu) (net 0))
 (segment (start 85.09 48.006) (end 85.598 48.006) (width 1.5) (layer B.Cu) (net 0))
 (segment (start 80.01 47.03) (end 81.026 48.046) (width 1.5) (layer B.Cu) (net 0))
 (segment (start 80.01 41.656) (end 80.01 47.03) (width 1.5) (layer B.Cu) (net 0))
 (segment (start 82.804 41.656) (end 85.09 39.37) (width 1.5) (layer F.Cu) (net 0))
 (segment (start 85.09 39.37) (end 87.63 39.37) (width 1.5) (layer F.Cu) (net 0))
 (segment (start 82.55 41.656) (end 82.804 41.656) (width 1.5) (layer F.Cu) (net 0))
 (segment (start 82.55 54.102) (end 81.026 52.578) (width 1.5) (layer F.Cu) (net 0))
 (segment (start 82.55 55.88) (end 82.55 54.102) (width 1.5) (layer F.Cu) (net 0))
 (segment (start 81.026 50.546) (end 81.026 52.578) (width 1.5) (layer F.Cu) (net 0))
 (segment (start 86.106 46.736) (end 86.106 43.434) (width 0.5) (layer B.Cu) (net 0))
 (segment (start 89.662 50.292) (end 86.106 46.736) (width 0.5) (layer B.Cu) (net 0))
 (segment (start 98.425 51.562) (end 98.425 50.927) (width 0.5) (layer B.Cu) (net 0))
 (segment (start 97.79 50.292) (end 89.662 50.292) (width 0.5) (layer B.Cu) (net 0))
 (segment (start 98.425 50.927) (end 97.79 50.292) (width 0.5) (layer B.Cu) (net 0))
 (segment (start 86.106 43.434) (end 87.63 41.91) (width 0.5) (layer B.Cu) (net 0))
 (segment (start 86.106 43.688) (end 86.106 43.434) (width 0.5) (layer B.Cu) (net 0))
 (segment (start 99.695 55.88) (end 99.695 44.704) (width 0.5) (layer B.Cu) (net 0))
 (segment (start 98.425 57.15) (end 99.695 55.88) (width 0.5) (layer B.Cu) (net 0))
 (segment (start 92.202 43.942) (end 90.17 41.91) (width 0.5) (layer B.Cu) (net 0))
 (segment (start 99.695 44.704) (end 98.933 43.942) (width 0.5) (layer B.Cu) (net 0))
 (segment (start 98.933 43.942) (end 92.202 43.942) (width 0.5) (layer B.Cu) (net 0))
 (segment (start 99.187 43.307) (end 96.647 43.307) (width 0.5) (layer B.Cu) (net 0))
 (segment (start 100.33 44.45) (end 99.187 43.307) (width 0.5) (layer B.Cu) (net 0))
 (segment (start 96.647 43.307) (end 95.25 41.91) (width 0.5) (layer B.Cu) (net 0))
 (segment (start 100.33 66.548) (end 100.33 44.45) (width 0.5) (layer B.Cu) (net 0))
 (segment (start 100.33 66.675) (end 100.33 66.548) (width 0.5) (layer B.Cu) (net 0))
 (segment (start 98.425 68.58) (end 100.33 66.675) (width 0.5) (layer B.Cu) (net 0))
 (segment (start 92.71 41.91) (end 94.742 43.942) (width 0.5) (layer F.Cu) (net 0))
 (segment (start 98.933 43.942) (end 99.695 44.704) (width 0.5) (layer F.Cu) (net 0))
 (segment (start 94.742 43.942) (end 98.933 43.942) (width 0.5) (layer F.Cu) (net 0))
 (segment (start 97.79 41.91) (end 100.33 44.45) (width 0.5) (layer F.Cu) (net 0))
 (segment (start 100.33 72.517) (end 98.425 74.422) (width 0.5) (layer F.Cu) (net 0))
 (segment (start 100.33 44.45) (end 100.33 72.517) (width 0.5) (layer F.Cu) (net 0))
 (segment (start 98.425 62.738) (end 99.695 61.468) (width 0.5) (layer F.Cu) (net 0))
 (segment (start 99.695 61.468) (end 99.695 44.831) (width 0.5) (layer F.Cu) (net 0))
 (segment (start 92.964 53.8845) (end 95.9215 53.8845) (width 0.25) (layer F.Cu) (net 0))
 (segment (start 97.155 55.118) (end 97.155 57.15) (width 0.25) (layer F.Cu) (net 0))
 (segment (start 95.9215 53.8845) (end 97.155 55.118) (width 0.25) (layer F.Cu) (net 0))
 (segment (start 92.2925 58.8375) (end 92.964 58.8375) (width 0.25) (layer F.Cu) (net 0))
 (segment (start 92.964 58.8375) (end 94.9055 58.8375) (width 0.25) (layer F.Cu) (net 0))
 (segment (start 97.155 61.087) (end 97.155 62.738) (width 0.25) (layer F.Cu) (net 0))
 (segment (start 94.9055 58.8375) (end 97.155 61.087) (width 0.25) (layer F.Cu) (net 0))
 (segment (start 90.17 63.5) (end 90.678 63.5) (width 0.25) (layer F.Cu) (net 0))
 (segment (start 90.17 66.04) (end 90.17 66.548) (width 0.25) (layer F.Cu) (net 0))
 (segment (start 92.3655 68.7435) (end 92.964 68.7435) (width 0.25) (layer F.Cu) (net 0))
 (segment (start 92.964 71.7185) (end 96.4835 71.7185) (width 0.25) (layer F.Cu) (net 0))
 (segment (start 97.155 72.39) (end 97.155 74.422) (width 0.25) (layer F.Cu) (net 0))
 (segment (start 96.4835 71.7185) (end 97.155 72.39) (width 0.25) (layer F.Cu) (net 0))
 (segment (start 90.3335 68.7435) (end 92.964 68.7435) (width 0.25) (layer F.Cu) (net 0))
 (segment (start 90.17 68.58) (end 90.3335 68.7435) (width 0.25) (layer F.Cu) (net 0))
 (segment (start 90.17 66.04) (end 90.551 66.04) (width 0.25) (layer F.Cu) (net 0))
 (segment (start 91.2765 66.7655) (end 92.964 66.7655) (width 0.25) (layer F.Cu) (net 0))
 (segment (start 90.551 66.04) (end 91.2765 66.7655) (width 0.25) (layer F.Cu) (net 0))
 (segment (start 97.155 66.548) (end 97.155 68.58) (width 0.25) (layer F.Cu) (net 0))
 (segment (start 94.361 63.754) (end 97.155 66.548) (width 0.25) (layer F.Cu) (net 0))
 (segment (start 93.0005 63.754) (end 92.964 63.7905) (width 0.25) (layer F.Cu) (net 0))
 (segment (start 94.361 63.754) (end 93.0005 63.754) (width 0.25) (layer F.Cu) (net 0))
 (segment (start 91.8575 61.8125) (end 92.964 61.8125) (width 0.25) (layer F.Cu) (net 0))
 (segment (start 90.17 63.5) (end 91.8575 61.8125) (width 0.25) (layer F.Cu) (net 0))
 (segment (start 92.2385 56.8595) (end 92.964 56.8595) (width 0.25) (layer F.Cu) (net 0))
 (segment (start 91.44 57.785) (end 92.2385 56.9865) (width 0.25) (layer F.Cu) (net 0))
 (segment (start 92.2385 51.9065) (end 92.964 51.9065) (width 0.25) (layer F.Cu) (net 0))
 (segment (start 91.44 57.15) (end 91.44 52.705) (width 0.25) (layer F.Cu) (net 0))
 (segment (start 91.44 52.705) (end 92.2385 51.9065) (width 0.25) (layer F.Cu) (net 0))
 (segment (start 91.44 59.69) (end 91.44 57.785) (width 0.25) (layer F.Cu) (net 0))
 (segment (start 90.17 60.96) (end 91.44 59.69) (width 0.25) (layer F.Cu) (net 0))
 (segment (start 82.55 55.198) (end 85.17 52.578) (width 1.5) (layer F.Cu) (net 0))
 (segment (start 82.55 55.88) (end 82.55 55.198) (width 1.5) (layer F.Cu) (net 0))
 (segment (start 85.17 52.578) (end 85.17 47.578) (width 1.5) (layer F.Cu) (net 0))
 (segment (start 85.17 47.578) (end 85.09 47.498) (width 1.5) (layer F.Cu) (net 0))
 (segment (start 82.55 46.482) (end 82.55 41.656) (width 1.5) (layer F.Cu) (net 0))
 (segment (start 82.931 46.863) (end 82.55 46.482) (width 1.5) (layer F.Cu) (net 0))
 (segment (start 92.583 45.72) (end 92.71 45.72) (width 0.25) (layer F.Cu) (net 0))
 (segment (start 87.63 50.546) (end 92.583 45.593) (width 0.25) (layer F.Cu) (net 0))
 (segment (start 96.139 47.371) (end 96.2025 47.3075) (width 0.25) (layer F.Cu) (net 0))
 (segment (start 96.139 47.371) (end 97.79 45.72) (width 0.25) (layer F.Cu) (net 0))
 (segment (start 90.17 47.371) (end 90.17 45.72) (width 0.25) (layer F.Cu) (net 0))
 (segment (start 87.122 56.388) (end 87.122 50.419) (width 0.25) (layer F.Cu) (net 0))
 (segment (start 82.55 60.96) (end 87.122 56.388) (width 0.25) (layer F.Cu) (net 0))
 (segment (start 87.63 60.96) (end 87.63 50.546) (width 0.25) (layer F.Cu) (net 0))
 (segment (start 82.55 66.04) (end 87.63 60.96) (width 0.25) (layer F.Cu) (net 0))
 (segment (start 92.075 47.371) (end 96.139 47.371) (width 0.25) (layer F.Cu) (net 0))
 (segment (start 88.646 50.8) (end 92.075 47.371) (width 0.25) (layer F.Cu) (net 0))
 (segment (start 82.55 71.12) (end 88.646 65.024) (width 0.25) (layer F.Cu) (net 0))
 (segment (start 88.646 65.024) (end 88.646 50.8) (width 0.25) (layer F.Cu) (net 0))
 (segment (start 93.98 46.99) (end 95.25 45.72) (width 0.25) (layer F.Cu) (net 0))
 (segment (start 91.821 46.99) (end 93.98 46.99) (width 0.25) (layer F.Cu) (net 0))
 (segment (start 82.55 68.58) (end 88.138 62.992) (width 0.25) (layer F.Cu) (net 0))
 (segment (start 88.138 50.673) (end 91.821 46.99) (width 0.25) (layer F.Cu) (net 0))
 (segment (start 88.138 62.992) (end 88.138 50.673) (width 0.25) (layer F.Cu) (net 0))
 (segment (start 82.55 66.04) (end 84.8725 66.04) (width 0.25) (layer B.Cu) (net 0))
 (segment (start 82.55 68.58) (end 84.8725 68.58) (width 0.25) (layer B.Cu) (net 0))
 (segment (start 82.55 71.12) (end 84.8725 71.12) (width 0.25) (layer B.Cu) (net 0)))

